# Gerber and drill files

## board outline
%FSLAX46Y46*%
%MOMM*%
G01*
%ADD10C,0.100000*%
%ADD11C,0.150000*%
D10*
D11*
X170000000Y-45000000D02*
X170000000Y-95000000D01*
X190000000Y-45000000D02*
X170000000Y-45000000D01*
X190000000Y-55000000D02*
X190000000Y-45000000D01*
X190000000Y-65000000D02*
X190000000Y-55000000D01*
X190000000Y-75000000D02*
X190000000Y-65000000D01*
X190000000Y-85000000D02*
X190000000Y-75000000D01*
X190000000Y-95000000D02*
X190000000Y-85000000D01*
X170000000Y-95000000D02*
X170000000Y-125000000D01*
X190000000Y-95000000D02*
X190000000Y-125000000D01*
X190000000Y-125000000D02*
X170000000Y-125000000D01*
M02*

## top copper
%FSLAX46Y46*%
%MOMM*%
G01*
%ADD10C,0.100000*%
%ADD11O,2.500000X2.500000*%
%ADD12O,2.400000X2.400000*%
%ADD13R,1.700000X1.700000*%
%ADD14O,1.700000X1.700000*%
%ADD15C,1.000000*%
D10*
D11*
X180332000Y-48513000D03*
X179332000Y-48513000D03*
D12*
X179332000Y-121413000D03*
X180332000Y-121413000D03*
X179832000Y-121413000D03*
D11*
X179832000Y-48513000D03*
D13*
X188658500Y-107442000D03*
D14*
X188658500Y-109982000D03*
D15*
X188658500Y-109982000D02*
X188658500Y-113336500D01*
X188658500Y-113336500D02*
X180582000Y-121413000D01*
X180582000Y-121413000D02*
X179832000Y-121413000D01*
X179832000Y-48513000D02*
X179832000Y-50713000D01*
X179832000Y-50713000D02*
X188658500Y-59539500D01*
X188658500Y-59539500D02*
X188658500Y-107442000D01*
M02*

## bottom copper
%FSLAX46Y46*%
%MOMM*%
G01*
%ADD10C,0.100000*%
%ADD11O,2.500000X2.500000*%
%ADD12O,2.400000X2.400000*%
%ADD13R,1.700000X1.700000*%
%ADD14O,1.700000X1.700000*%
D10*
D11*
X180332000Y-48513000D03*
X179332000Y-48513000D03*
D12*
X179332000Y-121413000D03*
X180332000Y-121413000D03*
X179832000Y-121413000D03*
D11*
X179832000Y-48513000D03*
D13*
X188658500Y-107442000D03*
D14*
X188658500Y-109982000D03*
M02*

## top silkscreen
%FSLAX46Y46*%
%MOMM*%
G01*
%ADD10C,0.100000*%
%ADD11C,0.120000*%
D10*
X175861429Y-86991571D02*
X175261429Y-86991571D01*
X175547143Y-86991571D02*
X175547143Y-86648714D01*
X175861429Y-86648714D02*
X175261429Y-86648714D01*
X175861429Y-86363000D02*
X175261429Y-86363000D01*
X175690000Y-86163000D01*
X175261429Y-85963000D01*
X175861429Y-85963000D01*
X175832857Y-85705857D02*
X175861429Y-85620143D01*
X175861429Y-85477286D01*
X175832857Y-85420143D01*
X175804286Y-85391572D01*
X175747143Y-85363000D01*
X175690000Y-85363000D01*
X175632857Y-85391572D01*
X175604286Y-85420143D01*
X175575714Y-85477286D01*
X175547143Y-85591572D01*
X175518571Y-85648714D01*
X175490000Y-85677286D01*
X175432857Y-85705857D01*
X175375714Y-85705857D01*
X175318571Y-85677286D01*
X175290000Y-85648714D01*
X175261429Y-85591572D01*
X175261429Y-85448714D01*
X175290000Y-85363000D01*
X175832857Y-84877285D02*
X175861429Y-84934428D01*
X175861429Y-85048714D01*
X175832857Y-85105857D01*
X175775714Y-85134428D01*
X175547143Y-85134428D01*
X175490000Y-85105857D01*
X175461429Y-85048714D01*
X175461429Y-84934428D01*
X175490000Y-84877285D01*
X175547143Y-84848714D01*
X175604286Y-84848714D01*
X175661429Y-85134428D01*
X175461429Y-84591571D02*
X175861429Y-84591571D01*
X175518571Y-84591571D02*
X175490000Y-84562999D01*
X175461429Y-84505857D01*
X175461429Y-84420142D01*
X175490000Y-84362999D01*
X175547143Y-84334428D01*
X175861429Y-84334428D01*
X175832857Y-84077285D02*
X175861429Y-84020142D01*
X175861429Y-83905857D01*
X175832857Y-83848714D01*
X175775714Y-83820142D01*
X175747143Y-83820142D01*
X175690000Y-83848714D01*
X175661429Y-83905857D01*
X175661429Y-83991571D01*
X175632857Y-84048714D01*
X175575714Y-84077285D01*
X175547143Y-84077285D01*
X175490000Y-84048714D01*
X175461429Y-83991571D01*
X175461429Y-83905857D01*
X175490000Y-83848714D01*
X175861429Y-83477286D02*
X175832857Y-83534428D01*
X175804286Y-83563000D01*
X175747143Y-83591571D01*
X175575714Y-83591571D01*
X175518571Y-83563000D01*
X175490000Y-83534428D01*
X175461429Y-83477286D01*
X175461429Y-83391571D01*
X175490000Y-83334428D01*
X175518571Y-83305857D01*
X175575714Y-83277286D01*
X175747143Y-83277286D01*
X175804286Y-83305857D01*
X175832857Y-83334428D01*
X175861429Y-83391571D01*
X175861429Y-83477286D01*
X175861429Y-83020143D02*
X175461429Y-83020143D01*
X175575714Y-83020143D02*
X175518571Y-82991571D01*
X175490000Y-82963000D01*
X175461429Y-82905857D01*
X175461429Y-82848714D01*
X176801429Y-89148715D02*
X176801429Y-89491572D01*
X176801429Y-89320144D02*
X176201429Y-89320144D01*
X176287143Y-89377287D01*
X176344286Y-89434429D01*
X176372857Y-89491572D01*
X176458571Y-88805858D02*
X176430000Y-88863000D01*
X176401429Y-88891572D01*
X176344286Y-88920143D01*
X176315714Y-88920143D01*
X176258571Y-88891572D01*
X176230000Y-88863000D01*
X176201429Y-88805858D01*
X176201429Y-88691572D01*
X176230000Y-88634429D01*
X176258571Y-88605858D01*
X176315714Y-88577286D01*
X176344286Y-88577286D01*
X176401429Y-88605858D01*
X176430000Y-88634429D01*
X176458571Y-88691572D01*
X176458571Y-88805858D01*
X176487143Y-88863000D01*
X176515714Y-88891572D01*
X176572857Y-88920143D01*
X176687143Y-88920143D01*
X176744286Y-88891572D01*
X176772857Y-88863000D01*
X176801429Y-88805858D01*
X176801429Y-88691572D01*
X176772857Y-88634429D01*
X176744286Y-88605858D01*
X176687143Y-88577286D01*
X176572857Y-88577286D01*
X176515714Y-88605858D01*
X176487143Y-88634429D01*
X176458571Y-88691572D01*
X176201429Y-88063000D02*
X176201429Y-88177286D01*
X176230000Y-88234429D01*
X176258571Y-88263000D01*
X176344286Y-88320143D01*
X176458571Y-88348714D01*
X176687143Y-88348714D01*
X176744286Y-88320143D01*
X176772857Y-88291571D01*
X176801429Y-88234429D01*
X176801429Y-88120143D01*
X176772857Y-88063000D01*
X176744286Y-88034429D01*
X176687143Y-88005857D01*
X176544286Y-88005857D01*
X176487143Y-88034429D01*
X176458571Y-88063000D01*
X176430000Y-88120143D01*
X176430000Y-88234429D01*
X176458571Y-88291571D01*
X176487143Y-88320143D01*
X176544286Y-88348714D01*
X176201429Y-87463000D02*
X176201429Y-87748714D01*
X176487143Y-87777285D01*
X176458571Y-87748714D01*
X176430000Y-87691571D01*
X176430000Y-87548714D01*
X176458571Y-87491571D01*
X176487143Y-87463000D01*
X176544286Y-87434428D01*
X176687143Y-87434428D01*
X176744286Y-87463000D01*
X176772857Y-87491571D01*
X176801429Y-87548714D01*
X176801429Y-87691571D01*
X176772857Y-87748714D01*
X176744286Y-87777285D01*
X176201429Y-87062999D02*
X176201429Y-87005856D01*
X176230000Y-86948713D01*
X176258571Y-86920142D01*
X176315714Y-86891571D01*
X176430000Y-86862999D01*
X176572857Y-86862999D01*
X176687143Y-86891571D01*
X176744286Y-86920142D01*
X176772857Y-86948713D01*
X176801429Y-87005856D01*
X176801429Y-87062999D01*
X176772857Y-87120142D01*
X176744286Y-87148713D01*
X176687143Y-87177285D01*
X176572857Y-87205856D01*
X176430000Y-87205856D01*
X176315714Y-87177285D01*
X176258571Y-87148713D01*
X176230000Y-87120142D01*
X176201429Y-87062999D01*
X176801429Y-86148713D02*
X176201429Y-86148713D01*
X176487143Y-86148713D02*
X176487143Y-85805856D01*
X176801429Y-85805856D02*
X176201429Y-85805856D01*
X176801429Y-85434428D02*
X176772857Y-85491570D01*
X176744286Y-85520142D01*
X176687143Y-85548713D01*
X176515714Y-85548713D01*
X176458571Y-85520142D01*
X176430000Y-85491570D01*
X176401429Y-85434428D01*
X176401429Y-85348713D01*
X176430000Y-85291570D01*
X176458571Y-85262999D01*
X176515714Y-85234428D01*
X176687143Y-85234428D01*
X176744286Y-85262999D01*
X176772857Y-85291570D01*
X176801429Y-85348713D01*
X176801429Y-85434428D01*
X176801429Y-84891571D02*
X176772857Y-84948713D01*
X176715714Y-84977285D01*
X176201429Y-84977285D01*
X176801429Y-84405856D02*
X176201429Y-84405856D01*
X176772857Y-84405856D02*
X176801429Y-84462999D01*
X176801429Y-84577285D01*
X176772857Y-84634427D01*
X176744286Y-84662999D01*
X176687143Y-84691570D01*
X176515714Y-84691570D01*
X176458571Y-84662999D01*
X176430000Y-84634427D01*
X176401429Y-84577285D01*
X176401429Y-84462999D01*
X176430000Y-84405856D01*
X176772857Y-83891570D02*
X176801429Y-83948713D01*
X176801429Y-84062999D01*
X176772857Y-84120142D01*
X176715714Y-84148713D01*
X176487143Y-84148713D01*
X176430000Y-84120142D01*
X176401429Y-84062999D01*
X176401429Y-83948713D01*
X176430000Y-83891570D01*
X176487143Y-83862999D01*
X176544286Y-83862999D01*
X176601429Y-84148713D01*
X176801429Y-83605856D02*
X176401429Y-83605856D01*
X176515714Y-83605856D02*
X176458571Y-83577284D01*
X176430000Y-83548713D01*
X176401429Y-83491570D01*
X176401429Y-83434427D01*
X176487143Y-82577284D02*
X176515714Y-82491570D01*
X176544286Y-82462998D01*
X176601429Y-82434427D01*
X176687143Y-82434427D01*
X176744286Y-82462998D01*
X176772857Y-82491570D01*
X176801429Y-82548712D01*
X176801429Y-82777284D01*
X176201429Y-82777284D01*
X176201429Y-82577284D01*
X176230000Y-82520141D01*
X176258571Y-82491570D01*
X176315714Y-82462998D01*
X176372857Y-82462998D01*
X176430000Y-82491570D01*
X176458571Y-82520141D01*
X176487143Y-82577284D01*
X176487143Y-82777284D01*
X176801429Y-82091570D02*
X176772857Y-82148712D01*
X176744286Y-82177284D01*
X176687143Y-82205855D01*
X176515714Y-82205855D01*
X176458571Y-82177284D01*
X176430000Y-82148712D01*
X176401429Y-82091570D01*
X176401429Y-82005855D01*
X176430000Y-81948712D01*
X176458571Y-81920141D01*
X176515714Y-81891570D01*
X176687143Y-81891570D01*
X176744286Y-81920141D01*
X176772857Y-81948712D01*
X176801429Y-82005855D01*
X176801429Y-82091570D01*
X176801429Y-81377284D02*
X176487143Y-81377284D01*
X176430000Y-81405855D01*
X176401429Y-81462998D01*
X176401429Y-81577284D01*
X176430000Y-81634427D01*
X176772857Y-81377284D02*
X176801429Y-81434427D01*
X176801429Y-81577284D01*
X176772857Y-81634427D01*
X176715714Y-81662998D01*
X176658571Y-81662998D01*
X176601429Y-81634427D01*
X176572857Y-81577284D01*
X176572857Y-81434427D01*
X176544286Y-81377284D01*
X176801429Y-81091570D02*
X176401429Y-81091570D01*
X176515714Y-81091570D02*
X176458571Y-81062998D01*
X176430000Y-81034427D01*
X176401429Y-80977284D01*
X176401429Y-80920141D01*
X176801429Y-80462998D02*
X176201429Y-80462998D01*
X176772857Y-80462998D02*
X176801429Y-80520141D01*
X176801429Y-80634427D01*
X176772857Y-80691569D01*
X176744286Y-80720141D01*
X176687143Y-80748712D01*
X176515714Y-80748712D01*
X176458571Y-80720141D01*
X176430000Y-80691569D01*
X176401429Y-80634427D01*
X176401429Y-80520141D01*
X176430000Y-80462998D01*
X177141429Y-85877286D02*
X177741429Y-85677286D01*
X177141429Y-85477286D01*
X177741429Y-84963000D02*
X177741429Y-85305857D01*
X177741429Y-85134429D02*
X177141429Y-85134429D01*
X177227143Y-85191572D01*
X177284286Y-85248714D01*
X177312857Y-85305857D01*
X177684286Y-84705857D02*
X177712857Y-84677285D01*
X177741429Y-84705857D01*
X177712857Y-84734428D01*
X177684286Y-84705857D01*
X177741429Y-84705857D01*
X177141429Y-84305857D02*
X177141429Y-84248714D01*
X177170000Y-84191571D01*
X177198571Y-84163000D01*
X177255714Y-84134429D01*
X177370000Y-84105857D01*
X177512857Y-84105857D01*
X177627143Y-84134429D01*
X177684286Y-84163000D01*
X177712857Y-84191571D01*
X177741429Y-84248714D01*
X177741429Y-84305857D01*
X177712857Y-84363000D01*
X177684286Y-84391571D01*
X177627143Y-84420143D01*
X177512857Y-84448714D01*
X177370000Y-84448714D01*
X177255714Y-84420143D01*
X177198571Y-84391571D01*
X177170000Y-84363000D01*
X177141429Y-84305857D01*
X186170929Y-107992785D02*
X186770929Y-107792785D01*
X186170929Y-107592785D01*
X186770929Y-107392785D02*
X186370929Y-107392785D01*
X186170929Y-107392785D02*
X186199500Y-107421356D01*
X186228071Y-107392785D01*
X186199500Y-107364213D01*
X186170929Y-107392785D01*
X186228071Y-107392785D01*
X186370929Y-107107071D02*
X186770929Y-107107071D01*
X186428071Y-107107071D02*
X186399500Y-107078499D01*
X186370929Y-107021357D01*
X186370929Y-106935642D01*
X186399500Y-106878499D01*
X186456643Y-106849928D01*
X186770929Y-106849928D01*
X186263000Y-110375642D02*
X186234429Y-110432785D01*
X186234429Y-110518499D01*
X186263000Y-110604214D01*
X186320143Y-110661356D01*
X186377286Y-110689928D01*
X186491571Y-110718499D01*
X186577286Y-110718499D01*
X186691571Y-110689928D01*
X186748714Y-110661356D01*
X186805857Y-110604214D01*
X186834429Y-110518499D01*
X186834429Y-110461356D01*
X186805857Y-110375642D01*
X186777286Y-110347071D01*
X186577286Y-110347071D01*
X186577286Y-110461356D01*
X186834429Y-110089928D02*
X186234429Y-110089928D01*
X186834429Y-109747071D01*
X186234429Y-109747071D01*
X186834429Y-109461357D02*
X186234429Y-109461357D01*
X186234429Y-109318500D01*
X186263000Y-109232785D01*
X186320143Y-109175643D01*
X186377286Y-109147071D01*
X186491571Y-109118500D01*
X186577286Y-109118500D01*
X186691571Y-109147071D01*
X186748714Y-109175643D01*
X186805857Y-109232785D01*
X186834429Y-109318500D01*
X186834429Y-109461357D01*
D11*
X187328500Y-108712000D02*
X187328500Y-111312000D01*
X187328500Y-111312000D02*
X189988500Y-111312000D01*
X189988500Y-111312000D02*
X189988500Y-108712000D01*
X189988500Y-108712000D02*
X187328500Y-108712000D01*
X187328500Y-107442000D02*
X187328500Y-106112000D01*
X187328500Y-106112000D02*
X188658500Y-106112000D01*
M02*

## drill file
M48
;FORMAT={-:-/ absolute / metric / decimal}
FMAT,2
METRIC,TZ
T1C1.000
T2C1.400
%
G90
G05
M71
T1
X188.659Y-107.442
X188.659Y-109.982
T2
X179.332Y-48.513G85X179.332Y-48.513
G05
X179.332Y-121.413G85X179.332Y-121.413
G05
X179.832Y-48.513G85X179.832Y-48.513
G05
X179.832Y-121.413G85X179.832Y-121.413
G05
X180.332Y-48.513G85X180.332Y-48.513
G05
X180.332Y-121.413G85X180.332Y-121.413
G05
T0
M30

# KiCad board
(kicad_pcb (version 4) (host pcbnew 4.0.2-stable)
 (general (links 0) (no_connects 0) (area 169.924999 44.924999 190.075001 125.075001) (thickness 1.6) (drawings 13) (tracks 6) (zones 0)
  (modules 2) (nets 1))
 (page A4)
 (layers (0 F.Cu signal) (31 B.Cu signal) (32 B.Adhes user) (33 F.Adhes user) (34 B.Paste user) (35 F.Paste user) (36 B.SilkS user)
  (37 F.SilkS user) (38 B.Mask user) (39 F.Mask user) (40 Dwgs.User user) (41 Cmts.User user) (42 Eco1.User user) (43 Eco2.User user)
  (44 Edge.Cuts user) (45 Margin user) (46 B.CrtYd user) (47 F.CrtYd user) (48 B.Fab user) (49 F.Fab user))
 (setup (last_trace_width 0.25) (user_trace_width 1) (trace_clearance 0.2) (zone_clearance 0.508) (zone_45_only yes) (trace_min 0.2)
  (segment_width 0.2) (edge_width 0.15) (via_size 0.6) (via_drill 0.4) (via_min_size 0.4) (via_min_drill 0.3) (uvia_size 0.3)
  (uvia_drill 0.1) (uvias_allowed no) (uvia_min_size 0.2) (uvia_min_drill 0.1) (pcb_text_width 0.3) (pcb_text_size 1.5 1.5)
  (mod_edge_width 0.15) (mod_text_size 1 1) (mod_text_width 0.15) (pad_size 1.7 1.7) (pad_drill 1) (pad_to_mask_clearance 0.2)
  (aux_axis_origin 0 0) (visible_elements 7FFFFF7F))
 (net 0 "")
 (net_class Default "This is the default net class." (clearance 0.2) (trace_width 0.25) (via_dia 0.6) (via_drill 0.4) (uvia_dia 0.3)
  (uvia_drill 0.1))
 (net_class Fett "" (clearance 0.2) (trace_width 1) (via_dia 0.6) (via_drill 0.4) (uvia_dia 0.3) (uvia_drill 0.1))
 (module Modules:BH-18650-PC (layer B.Cu) (at 179.832 84.963)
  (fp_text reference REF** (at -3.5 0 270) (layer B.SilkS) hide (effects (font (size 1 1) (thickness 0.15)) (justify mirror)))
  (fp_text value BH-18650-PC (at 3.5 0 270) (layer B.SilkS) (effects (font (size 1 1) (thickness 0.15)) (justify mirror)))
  (pad 2 thru_hole oval (at 0.5 -36.45) (size 2.5 2.5) (drill oval 1.4) (layers *.Cu *.Mask B.SilkS))
  (pad 2 thru_hole oval (at -0.5 -36.45) (size 2.5 2.5) (drill oval 1.4) (layers *.Cu *.Mask B.SilkS))
  (pad 1 thru_hole oval (at -0.5 36.45) (size 2.4 2.4) (drill oval 1.4) (layers *.Cu *.Mask B.SilkS))
  (pad 1 thru_hole oval (at 0.5 36.45) (size 2.4 2.4) (drill oval 1.4) (layers *.Cu *.Mask B.SilkS))
  (pad 1 thru_hole oval (at 0 36.45) (size 2.4 2.4) (drill oval 1.4) (layers *.Cu *.Mask B.SilkS))
  (pad 2 thru_hole oval (at 0 -36.45) (size 2.5 2.5) (drill oval 1.4) (layers *.Cu *.Mask B.SilkS)))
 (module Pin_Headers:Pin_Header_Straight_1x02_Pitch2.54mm (layer F.Cu) (at 188.6585 107.442)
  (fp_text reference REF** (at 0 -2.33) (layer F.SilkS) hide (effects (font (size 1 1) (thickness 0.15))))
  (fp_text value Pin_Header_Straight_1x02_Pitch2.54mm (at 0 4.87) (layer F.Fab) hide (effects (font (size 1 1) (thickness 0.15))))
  (fp_line (start -1.33 1.27) (end -1.33 3.87) (layer F.SilkS) (width 0.12))
  (fp_line (start -1.33 3.87) (end 1.33 3.87) (layer F.SilkS) (width 0.12))
  (fp_line (start 1.33 3.87) (end 1.33 1.27) (layer F.SilkS) (width 0.12))
  (fp_line (start 1.33 1.27) (end -1.33 1.27) (layer F.SilkS) (width 0.12))
  (fp_line (start -1.33 0) (end -1.33 -1.33) (layer F.SilkS) (width 0.12))
  (fp_line (start -1.33 -1.33) (end 0 -1.33) (layer F.SilkS) (width 0.12))
  (pad 1 thru_hole rect (at 0 0) (size 1.7 1.7) (drill 1) (layers *.Cu *.Mask))
  (pad 2 thru_hole oval (at 0 2.54) (size 1.7 1.7) (drill 1) (layers *.Cu *.Mask)))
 (gr_line (start 170 45) (end 170 95) (angle 90) (layer Edge.Cuts) (width 0.15))
 (gr_line (start 190 45) (end 170 45) (angle 90) (layer Edge.Cuts) (width 0.15))
 (gr_line (start 190 55) (end 190 45) (angle 90) (layer Edge.Cuts) (width 0.15))
 (gr_line (start 190 65) (end 190 55) (angle 90) (layer Edge.Cuts) (width 0.15))
 (gr_line (start 190 75) (end 190 65) (angle 90) (layer Edge.Cuts) (width 0.15))
 (gr_line (start 190 85) (end 190 75) (angle 90) (layer Edge.Cuts) (width 0.15))
 (gr_line (start 190 95) (end 190 85) (angle 90) (layer Edge.Cuts) (width 0.15))
 (gr_line (start 170 95) (end 170 125) (angle 90) (layer Edge.Cuts) (width 0.15))
 (gr_line (start 190 95) (end 190 125) (angle 90) (layer Edge.Cuts) (width 0.15))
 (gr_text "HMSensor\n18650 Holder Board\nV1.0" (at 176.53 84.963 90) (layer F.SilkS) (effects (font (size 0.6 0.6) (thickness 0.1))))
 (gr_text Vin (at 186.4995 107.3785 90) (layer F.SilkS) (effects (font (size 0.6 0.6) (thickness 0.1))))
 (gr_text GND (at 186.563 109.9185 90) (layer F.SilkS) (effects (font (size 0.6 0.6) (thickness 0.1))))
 (gr_line (start 190 125) (end 170 125) (angle 90) (layer Edge.Cuts) (width 0.15))
 (segment (start 188.6585 109.982) (end 188.6585 113.3365) (width 1) (layer F.Cu) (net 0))
 (segment (start 188.6585 113.3365) (end 180.582 121.413) (width 1) (layer F.Cu) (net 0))
 (segment (start 180.582 121.413) (end 179.832 121.413) (width 1) (layer F.Cu) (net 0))
 (segment (start 179.832 48.513) (end 179.832 50.713) (width 1) (layer F.Cu) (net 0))
 (segment (start 179.832 50.713) (end 188.6585 59.5395) (width 1) (layer F.Cu) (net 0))
 (segment (start 188.6585 59.5395) (end 188.6585 107.442) (width 1) (layer F.Cu) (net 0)))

